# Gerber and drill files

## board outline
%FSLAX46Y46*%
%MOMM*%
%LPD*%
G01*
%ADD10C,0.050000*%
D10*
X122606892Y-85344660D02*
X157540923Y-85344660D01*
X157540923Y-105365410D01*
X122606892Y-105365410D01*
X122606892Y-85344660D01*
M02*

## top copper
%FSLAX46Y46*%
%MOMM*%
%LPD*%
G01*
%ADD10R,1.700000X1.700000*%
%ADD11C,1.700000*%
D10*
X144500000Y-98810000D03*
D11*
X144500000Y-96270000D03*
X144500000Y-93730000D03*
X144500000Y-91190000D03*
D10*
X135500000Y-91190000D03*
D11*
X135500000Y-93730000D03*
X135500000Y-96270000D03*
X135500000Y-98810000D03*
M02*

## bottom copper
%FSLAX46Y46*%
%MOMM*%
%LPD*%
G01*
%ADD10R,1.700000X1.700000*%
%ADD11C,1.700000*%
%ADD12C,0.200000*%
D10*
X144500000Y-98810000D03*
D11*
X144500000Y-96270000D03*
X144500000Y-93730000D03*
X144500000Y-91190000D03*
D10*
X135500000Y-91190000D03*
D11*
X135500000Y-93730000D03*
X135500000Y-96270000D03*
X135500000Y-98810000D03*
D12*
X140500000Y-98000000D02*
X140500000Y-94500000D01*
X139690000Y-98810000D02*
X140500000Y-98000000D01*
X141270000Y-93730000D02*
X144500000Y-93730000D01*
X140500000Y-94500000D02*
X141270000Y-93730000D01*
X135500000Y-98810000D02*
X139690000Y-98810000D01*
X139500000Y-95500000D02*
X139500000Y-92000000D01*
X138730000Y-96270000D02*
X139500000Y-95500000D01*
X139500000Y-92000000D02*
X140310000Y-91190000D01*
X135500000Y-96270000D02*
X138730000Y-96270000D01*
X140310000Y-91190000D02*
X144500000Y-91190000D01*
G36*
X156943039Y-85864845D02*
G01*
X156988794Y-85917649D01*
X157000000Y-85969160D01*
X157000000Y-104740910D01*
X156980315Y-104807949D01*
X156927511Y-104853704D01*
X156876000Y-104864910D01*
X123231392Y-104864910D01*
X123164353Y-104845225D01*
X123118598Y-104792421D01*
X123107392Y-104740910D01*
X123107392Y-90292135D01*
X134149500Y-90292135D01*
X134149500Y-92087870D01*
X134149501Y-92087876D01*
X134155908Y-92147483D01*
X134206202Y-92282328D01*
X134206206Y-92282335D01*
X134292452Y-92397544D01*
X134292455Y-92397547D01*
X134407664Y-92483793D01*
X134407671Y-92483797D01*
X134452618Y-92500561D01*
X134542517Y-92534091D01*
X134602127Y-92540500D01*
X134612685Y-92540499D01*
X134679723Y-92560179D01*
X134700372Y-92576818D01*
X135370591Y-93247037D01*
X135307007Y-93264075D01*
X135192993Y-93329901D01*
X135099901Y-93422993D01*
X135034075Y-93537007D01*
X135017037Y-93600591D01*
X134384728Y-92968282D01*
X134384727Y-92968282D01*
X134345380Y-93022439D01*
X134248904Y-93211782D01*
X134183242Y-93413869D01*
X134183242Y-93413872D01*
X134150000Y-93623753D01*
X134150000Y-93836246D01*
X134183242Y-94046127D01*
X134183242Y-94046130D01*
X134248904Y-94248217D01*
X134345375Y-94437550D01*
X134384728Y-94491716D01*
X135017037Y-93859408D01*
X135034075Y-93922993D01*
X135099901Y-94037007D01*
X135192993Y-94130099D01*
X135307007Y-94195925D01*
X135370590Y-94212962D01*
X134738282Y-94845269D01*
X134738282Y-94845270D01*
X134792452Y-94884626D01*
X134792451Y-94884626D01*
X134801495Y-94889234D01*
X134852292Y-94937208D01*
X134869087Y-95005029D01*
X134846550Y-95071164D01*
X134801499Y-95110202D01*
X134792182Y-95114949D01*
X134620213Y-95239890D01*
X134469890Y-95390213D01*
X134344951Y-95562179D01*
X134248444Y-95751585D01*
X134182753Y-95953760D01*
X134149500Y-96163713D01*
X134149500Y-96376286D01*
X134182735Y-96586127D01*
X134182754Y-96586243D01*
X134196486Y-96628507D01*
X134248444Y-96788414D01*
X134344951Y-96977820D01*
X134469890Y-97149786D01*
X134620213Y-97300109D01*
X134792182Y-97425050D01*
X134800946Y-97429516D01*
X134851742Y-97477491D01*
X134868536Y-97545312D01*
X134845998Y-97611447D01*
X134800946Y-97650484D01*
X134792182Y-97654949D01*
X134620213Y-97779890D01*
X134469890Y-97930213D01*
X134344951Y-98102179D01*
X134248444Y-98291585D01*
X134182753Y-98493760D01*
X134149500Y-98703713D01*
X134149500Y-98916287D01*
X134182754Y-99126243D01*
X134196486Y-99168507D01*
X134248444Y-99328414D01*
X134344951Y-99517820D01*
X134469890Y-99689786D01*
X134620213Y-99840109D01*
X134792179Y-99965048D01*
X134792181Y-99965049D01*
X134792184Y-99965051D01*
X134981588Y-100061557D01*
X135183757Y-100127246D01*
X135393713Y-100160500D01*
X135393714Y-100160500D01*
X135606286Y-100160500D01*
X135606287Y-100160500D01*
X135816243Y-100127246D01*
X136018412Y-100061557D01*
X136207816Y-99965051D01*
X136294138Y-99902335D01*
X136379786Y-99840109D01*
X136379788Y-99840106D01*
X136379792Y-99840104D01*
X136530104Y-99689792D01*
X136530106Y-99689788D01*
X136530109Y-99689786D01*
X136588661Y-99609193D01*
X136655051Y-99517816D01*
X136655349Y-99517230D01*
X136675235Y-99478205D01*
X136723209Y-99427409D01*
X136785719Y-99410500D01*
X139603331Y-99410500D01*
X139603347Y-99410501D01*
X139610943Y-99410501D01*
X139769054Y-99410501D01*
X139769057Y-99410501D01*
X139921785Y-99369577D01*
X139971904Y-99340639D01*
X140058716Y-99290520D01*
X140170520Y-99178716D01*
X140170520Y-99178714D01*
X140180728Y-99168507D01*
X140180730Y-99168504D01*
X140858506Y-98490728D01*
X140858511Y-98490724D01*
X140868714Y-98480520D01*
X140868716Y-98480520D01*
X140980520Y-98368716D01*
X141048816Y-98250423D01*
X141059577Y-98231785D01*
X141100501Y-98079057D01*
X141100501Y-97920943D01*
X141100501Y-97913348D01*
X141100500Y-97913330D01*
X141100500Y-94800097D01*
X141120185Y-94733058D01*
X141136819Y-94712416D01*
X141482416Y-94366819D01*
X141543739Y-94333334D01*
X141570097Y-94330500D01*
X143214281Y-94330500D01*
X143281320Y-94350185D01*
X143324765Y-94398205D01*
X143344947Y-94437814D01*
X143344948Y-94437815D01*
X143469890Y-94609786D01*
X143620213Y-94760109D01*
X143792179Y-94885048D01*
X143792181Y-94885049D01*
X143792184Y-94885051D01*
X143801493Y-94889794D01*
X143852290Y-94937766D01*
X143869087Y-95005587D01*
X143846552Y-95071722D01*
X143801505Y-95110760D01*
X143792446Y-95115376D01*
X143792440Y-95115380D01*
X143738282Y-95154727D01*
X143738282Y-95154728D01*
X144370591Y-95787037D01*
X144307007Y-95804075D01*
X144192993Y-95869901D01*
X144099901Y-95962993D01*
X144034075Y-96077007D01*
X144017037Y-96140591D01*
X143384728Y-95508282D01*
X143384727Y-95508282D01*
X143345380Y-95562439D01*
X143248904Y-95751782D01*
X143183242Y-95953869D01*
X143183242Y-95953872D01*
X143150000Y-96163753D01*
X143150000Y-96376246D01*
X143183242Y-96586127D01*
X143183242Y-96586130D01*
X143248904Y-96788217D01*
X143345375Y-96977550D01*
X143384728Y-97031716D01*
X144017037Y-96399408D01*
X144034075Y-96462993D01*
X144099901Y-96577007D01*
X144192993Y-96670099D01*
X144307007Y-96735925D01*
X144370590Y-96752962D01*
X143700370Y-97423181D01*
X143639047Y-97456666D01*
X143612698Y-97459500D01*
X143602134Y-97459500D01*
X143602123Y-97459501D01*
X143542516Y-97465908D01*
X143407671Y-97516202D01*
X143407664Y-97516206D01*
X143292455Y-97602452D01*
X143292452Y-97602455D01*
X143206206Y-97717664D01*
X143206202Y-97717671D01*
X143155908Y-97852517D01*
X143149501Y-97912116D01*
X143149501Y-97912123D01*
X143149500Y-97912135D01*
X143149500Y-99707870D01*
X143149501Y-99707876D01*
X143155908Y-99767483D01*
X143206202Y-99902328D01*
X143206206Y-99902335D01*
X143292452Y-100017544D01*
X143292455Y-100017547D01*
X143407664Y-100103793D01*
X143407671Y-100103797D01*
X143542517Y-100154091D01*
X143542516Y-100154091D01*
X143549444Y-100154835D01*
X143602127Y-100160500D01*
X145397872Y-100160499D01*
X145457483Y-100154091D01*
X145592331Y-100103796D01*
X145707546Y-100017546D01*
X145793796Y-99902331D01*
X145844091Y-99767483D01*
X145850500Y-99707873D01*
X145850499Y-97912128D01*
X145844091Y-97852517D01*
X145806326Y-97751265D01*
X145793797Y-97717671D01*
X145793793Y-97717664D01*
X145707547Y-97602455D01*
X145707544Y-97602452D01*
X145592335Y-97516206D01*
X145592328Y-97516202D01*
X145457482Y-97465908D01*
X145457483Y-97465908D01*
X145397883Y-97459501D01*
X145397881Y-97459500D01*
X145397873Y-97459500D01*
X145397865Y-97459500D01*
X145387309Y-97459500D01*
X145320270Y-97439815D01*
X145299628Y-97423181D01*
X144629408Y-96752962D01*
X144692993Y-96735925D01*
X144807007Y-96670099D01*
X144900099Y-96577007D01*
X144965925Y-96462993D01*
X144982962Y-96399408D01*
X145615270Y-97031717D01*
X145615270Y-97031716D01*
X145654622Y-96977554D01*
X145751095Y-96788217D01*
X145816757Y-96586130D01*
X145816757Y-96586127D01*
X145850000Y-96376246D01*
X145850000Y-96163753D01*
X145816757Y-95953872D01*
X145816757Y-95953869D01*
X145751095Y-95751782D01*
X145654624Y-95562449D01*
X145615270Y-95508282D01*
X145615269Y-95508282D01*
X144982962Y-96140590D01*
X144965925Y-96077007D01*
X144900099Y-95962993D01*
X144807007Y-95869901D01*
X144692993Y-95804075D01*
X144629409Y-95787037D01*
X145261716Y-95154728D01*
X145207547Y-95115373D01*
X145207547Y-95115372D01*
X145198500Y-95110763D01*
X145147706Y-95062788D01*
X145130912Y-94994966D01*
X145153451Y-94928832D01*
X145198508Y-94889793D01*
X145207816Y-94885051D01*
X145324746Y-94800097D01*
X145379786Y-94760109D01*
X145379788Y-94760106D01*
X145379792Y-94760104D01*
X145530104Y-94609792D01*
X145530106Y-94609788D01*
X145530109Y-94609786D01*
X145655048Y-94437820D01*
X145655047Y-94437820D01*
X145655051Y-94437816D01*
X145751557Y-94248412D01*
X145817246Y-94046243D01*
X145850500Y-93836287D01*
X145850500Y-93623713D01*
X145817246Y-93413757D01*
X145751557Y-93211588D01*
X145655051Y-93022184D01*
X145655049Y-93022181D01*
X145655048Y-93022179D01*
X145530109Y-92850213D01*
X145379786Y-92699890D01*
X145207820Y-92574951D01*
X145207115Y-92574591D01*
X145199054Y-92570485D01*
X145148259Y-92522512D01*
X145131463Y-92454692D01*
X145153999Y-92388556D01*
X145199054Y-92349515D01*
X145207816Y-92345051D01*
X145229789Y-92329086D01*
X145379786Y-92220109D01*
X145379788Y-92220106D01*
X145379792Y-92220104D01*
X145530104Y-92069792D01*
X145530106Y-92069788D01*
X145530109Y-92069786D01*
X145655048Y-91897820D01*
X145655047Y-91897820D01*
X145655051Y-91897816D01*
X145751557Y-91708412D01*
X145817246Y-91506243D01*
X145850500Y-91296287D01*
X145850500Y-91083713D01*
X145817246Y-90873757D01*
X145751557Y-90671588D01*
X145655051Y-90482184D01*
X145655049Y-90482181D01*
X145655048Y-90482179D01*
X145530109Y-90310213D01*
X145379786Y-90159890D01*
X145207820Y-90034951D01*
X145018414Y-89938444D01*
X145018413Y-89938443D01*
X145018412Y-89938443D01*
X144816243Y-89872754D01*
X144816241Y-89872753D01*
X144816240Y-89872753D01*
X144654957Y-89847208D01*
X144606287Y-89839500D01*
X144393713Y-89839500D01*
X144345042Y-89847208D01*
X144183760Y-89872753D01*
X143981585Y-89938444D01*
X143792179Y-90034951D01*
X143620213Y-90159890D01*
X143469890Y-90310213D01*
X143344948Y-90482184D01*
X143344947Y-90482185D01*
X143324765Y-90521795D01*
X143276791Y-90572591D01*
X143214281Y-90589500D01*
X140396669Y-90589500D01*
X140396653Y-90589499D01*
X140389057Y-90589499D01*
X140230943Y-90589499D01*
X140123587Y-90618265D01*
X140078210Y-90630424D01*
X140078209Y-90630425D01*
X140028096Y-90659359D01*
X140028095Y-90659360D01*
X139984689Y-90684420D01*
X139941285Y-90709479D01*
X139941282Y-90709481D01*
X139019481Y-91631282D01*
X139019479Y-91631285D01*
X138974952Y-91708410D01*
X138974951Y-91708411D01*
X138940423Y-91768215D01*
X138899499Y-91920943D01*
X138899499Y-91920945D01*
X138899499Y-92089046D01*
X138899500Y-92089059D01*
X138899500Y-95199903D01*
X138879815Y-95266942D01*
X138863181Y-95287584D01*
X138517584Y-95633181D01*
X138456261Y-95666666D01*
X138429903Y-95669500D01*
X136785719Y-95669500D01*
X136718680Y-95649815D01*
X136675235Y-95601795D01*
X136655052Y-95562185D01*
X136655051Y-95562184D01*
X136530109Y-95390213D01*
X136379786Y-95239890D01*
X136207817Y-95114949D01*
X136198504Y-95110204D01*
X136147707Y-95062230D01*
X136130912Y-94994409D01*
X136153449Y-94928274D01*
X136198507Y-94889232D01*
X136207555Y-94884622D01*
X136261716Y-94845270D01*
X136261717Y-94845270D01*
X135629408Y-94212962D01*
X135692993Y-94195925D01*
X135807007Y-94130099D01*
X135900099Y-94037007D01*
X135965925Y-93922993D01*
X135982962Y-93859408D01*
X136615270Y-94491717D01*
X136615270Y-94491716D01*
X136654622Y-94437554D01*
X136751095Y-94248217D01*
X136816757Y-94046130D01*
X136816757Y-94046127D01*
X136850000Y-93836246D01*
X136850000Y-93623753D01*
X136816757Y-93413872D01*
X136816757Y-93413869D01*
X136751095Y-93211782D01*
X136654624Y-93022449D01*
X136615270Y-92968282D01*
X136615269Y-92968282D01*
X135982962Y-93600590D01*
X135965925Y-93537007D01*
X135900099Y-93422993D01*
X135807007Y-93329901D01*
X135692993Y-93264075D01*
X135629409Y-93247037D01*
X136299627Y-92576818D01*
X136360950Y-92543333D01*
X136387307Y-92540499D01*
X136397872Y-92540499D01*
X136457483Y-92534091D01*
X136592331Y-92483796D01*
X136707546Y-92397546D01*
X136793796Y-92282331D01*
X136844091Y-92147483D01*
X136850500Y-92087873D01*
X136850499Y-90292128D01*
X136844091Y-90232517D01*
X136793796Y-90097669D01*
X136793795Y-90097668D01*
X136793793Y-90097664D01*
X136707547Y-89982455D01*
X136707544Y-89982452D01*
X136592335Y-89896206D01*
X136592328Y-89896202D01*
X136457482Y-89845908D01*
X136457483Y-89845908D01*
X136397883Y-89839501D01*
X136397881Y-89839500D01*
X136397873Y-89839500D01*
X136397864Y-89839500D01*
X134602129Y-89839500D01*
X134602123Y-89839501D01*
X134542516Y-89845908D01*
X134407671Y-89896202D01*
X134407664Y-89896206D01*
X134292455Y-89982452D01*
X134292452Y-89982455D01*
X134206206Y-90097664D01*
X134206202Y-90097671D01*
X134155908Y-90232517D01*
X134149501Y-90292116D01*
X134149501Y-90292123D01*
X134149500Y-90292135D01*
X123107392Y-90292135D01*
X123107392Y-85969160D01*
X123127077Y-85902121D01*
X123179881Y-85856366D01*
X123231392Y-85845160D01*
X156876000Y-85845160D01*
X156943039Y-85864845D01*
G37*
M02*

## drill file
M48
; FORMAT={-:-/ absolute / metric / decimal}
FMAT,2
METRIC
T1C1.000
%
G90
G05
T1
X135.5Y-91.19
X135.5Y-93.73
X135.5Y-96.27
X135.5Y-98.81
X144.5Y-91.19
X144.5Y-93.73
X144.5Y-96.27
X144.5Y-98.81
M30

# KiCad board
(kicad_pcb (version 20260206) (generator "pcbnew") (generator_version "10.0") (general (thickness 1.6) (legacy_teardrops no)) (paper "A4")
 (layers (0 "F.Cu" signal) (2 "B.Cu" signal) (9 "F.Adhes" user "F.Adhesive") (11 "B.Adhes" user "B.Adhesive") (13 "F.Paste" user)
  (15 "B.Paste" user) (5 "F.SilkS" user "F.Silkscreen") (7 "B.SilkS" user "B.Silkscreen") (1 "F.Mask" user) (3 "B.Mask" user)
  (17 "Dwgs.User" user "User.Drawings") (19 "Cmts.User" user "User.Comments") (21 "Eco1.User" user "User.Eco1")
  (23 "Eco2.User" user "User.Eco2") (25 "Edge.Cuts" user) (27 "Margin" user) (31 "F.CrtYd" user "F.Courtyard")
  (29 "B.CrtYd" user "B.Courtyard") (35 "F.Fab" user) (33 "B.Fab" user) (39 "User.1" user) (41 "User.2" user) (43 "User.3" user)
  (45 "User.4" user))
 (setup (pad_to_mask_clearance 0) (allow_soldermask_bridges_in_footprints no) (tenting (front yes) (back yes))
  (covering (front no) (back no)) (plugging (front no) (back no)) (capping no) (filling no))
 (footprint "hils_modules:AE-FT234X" (layer "F.Cu") (at 149 95 90)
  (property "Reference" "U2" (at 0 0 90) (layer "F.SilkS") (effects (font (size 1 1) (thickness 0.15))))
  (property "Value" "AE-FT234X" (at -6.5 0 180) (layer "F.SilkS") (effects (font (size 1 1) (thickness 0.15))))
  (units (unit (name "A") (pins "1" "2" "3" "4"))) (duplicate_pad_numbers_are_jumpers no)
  (pad "1" thru_hole rect (at -3.81 -4.5 90) (size 1.7 1.7) (drill 1) (layers "*.Cu" "*.Mask") (remove_unused_layers no)
   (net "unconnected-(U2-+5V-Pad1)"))
  (pad "2" thru_hole circle (at -1.27 -4.5 90) (size 1.7 1.7) (drill 1) (layers "*.Cu" "*.Mask") (remove_unused_layers no) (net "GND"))
  (pad "3" thru_hole circle (at 1.27 -4.5 90) (size 1.7 1.7) (drill 1) (layers "*.Cu" "*.Mask") (remove_unused_layers no)
   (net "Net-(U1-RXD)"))
  (pad "4" thru_hole circle (at 3.81 -4.5 90) (size 1.7 1.7) (drill 1) (layers "*.Cu" "*.Mask") (remove_unused_layers no)
   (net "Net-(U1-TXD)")))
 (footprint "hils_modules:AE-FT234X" (layer "F.Cu") (at 131 95 -90)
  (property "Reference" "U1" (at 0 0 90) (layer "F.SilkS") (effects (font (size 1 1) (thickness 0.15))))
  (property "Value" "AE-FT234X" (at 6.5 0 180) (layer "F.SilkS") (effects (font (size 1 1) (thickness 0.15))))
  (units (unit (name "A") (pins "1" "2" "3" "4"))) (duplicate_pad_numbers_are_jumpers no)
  (pad "1" thru_hole rect (at -3.81 -4.5 270) (size 1.7 1.7) (drill 1) (layers "*.Cu" "*.Mask") (remove_unused_layers no)
   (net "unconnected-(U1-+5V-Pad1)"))
  (pad "2" thru_hole circle (at -1.27 -4.5 270) (size 1.7 1.7) (drill 1) (layers "*.Cu" "*.Mask") (remove_unused_layers no) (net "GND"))
  (pad "3" thru_hole circle (at 1.27 -4.5 270) (size 1.7 1.7) (drill 1) (layers "*.Cu" "*.Mask") (remove_unused_layers no)
   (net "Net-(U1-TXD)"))
  (pad "4" thru_hole circle (at 3.81 -4.5 270) (size 1.7 1.7) (drill 1) (layers "*.Cu" "*.Mask") (remove_unused_layers no)
   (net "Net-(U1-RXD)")))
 (gr_rect (start 122.606892 85.34466) (end 157.540923 105.36541) (stroke (width 0.05) (type default)) (fill no) (layer "Edge.Cuts"))
 (segment (start 140.5 98) (end 140.5 94.5) (width 0.2) (layer "B.Cu") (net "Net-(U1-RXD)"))
 (segment (start 139.69 98.81) (end 140.5 98) (width 0.2) (layer "B.Cu") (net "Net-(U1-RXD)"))
 (segment (start 141.27 93.73) (end 144.5 93.73) (width 0.2) (layer "B.Cu") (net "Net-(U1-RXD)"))
 (segment (start 140.5 94.5) (end 141.27 93.73) (width 0.2) (layer "B.Cu") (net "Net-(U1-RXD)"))
 (segment (start 135.5 98.81) (end 139.69 98.81) (width 0.2) (layer "B.Cu") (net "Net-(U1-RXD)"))
 (segment (start 139.5 95.5) (end 139.5 92) (width 0.2) (layer "B.Cu") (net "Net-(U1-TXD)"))
 (segment (start 138.73 96.27) (end 139.5 95.5) (width 0.2) (layer "B.Cu") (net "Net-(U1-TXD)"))
 (segment (start 139.5 92) (end 140.31 91.19) (width 0.2) (layer "B.Cu") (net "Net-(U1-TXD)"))
 (segment (start 135.5 96.27) (end 138.73 96.27) (width 0.2) (layer "B.Cu") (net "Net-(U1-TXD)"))
 (segment (start 140.31 91.19) (end 144.5 91.19) (width 0.2) (layer "B.Cu") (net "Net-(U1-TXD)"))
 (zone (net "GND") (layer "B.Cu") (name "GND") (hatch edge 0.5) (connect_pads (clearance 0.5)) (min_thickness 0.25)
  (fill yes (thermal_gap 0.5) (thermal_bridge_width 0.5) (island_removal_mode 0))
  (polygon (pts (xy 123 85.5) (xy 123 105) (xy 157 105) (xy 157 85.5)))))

